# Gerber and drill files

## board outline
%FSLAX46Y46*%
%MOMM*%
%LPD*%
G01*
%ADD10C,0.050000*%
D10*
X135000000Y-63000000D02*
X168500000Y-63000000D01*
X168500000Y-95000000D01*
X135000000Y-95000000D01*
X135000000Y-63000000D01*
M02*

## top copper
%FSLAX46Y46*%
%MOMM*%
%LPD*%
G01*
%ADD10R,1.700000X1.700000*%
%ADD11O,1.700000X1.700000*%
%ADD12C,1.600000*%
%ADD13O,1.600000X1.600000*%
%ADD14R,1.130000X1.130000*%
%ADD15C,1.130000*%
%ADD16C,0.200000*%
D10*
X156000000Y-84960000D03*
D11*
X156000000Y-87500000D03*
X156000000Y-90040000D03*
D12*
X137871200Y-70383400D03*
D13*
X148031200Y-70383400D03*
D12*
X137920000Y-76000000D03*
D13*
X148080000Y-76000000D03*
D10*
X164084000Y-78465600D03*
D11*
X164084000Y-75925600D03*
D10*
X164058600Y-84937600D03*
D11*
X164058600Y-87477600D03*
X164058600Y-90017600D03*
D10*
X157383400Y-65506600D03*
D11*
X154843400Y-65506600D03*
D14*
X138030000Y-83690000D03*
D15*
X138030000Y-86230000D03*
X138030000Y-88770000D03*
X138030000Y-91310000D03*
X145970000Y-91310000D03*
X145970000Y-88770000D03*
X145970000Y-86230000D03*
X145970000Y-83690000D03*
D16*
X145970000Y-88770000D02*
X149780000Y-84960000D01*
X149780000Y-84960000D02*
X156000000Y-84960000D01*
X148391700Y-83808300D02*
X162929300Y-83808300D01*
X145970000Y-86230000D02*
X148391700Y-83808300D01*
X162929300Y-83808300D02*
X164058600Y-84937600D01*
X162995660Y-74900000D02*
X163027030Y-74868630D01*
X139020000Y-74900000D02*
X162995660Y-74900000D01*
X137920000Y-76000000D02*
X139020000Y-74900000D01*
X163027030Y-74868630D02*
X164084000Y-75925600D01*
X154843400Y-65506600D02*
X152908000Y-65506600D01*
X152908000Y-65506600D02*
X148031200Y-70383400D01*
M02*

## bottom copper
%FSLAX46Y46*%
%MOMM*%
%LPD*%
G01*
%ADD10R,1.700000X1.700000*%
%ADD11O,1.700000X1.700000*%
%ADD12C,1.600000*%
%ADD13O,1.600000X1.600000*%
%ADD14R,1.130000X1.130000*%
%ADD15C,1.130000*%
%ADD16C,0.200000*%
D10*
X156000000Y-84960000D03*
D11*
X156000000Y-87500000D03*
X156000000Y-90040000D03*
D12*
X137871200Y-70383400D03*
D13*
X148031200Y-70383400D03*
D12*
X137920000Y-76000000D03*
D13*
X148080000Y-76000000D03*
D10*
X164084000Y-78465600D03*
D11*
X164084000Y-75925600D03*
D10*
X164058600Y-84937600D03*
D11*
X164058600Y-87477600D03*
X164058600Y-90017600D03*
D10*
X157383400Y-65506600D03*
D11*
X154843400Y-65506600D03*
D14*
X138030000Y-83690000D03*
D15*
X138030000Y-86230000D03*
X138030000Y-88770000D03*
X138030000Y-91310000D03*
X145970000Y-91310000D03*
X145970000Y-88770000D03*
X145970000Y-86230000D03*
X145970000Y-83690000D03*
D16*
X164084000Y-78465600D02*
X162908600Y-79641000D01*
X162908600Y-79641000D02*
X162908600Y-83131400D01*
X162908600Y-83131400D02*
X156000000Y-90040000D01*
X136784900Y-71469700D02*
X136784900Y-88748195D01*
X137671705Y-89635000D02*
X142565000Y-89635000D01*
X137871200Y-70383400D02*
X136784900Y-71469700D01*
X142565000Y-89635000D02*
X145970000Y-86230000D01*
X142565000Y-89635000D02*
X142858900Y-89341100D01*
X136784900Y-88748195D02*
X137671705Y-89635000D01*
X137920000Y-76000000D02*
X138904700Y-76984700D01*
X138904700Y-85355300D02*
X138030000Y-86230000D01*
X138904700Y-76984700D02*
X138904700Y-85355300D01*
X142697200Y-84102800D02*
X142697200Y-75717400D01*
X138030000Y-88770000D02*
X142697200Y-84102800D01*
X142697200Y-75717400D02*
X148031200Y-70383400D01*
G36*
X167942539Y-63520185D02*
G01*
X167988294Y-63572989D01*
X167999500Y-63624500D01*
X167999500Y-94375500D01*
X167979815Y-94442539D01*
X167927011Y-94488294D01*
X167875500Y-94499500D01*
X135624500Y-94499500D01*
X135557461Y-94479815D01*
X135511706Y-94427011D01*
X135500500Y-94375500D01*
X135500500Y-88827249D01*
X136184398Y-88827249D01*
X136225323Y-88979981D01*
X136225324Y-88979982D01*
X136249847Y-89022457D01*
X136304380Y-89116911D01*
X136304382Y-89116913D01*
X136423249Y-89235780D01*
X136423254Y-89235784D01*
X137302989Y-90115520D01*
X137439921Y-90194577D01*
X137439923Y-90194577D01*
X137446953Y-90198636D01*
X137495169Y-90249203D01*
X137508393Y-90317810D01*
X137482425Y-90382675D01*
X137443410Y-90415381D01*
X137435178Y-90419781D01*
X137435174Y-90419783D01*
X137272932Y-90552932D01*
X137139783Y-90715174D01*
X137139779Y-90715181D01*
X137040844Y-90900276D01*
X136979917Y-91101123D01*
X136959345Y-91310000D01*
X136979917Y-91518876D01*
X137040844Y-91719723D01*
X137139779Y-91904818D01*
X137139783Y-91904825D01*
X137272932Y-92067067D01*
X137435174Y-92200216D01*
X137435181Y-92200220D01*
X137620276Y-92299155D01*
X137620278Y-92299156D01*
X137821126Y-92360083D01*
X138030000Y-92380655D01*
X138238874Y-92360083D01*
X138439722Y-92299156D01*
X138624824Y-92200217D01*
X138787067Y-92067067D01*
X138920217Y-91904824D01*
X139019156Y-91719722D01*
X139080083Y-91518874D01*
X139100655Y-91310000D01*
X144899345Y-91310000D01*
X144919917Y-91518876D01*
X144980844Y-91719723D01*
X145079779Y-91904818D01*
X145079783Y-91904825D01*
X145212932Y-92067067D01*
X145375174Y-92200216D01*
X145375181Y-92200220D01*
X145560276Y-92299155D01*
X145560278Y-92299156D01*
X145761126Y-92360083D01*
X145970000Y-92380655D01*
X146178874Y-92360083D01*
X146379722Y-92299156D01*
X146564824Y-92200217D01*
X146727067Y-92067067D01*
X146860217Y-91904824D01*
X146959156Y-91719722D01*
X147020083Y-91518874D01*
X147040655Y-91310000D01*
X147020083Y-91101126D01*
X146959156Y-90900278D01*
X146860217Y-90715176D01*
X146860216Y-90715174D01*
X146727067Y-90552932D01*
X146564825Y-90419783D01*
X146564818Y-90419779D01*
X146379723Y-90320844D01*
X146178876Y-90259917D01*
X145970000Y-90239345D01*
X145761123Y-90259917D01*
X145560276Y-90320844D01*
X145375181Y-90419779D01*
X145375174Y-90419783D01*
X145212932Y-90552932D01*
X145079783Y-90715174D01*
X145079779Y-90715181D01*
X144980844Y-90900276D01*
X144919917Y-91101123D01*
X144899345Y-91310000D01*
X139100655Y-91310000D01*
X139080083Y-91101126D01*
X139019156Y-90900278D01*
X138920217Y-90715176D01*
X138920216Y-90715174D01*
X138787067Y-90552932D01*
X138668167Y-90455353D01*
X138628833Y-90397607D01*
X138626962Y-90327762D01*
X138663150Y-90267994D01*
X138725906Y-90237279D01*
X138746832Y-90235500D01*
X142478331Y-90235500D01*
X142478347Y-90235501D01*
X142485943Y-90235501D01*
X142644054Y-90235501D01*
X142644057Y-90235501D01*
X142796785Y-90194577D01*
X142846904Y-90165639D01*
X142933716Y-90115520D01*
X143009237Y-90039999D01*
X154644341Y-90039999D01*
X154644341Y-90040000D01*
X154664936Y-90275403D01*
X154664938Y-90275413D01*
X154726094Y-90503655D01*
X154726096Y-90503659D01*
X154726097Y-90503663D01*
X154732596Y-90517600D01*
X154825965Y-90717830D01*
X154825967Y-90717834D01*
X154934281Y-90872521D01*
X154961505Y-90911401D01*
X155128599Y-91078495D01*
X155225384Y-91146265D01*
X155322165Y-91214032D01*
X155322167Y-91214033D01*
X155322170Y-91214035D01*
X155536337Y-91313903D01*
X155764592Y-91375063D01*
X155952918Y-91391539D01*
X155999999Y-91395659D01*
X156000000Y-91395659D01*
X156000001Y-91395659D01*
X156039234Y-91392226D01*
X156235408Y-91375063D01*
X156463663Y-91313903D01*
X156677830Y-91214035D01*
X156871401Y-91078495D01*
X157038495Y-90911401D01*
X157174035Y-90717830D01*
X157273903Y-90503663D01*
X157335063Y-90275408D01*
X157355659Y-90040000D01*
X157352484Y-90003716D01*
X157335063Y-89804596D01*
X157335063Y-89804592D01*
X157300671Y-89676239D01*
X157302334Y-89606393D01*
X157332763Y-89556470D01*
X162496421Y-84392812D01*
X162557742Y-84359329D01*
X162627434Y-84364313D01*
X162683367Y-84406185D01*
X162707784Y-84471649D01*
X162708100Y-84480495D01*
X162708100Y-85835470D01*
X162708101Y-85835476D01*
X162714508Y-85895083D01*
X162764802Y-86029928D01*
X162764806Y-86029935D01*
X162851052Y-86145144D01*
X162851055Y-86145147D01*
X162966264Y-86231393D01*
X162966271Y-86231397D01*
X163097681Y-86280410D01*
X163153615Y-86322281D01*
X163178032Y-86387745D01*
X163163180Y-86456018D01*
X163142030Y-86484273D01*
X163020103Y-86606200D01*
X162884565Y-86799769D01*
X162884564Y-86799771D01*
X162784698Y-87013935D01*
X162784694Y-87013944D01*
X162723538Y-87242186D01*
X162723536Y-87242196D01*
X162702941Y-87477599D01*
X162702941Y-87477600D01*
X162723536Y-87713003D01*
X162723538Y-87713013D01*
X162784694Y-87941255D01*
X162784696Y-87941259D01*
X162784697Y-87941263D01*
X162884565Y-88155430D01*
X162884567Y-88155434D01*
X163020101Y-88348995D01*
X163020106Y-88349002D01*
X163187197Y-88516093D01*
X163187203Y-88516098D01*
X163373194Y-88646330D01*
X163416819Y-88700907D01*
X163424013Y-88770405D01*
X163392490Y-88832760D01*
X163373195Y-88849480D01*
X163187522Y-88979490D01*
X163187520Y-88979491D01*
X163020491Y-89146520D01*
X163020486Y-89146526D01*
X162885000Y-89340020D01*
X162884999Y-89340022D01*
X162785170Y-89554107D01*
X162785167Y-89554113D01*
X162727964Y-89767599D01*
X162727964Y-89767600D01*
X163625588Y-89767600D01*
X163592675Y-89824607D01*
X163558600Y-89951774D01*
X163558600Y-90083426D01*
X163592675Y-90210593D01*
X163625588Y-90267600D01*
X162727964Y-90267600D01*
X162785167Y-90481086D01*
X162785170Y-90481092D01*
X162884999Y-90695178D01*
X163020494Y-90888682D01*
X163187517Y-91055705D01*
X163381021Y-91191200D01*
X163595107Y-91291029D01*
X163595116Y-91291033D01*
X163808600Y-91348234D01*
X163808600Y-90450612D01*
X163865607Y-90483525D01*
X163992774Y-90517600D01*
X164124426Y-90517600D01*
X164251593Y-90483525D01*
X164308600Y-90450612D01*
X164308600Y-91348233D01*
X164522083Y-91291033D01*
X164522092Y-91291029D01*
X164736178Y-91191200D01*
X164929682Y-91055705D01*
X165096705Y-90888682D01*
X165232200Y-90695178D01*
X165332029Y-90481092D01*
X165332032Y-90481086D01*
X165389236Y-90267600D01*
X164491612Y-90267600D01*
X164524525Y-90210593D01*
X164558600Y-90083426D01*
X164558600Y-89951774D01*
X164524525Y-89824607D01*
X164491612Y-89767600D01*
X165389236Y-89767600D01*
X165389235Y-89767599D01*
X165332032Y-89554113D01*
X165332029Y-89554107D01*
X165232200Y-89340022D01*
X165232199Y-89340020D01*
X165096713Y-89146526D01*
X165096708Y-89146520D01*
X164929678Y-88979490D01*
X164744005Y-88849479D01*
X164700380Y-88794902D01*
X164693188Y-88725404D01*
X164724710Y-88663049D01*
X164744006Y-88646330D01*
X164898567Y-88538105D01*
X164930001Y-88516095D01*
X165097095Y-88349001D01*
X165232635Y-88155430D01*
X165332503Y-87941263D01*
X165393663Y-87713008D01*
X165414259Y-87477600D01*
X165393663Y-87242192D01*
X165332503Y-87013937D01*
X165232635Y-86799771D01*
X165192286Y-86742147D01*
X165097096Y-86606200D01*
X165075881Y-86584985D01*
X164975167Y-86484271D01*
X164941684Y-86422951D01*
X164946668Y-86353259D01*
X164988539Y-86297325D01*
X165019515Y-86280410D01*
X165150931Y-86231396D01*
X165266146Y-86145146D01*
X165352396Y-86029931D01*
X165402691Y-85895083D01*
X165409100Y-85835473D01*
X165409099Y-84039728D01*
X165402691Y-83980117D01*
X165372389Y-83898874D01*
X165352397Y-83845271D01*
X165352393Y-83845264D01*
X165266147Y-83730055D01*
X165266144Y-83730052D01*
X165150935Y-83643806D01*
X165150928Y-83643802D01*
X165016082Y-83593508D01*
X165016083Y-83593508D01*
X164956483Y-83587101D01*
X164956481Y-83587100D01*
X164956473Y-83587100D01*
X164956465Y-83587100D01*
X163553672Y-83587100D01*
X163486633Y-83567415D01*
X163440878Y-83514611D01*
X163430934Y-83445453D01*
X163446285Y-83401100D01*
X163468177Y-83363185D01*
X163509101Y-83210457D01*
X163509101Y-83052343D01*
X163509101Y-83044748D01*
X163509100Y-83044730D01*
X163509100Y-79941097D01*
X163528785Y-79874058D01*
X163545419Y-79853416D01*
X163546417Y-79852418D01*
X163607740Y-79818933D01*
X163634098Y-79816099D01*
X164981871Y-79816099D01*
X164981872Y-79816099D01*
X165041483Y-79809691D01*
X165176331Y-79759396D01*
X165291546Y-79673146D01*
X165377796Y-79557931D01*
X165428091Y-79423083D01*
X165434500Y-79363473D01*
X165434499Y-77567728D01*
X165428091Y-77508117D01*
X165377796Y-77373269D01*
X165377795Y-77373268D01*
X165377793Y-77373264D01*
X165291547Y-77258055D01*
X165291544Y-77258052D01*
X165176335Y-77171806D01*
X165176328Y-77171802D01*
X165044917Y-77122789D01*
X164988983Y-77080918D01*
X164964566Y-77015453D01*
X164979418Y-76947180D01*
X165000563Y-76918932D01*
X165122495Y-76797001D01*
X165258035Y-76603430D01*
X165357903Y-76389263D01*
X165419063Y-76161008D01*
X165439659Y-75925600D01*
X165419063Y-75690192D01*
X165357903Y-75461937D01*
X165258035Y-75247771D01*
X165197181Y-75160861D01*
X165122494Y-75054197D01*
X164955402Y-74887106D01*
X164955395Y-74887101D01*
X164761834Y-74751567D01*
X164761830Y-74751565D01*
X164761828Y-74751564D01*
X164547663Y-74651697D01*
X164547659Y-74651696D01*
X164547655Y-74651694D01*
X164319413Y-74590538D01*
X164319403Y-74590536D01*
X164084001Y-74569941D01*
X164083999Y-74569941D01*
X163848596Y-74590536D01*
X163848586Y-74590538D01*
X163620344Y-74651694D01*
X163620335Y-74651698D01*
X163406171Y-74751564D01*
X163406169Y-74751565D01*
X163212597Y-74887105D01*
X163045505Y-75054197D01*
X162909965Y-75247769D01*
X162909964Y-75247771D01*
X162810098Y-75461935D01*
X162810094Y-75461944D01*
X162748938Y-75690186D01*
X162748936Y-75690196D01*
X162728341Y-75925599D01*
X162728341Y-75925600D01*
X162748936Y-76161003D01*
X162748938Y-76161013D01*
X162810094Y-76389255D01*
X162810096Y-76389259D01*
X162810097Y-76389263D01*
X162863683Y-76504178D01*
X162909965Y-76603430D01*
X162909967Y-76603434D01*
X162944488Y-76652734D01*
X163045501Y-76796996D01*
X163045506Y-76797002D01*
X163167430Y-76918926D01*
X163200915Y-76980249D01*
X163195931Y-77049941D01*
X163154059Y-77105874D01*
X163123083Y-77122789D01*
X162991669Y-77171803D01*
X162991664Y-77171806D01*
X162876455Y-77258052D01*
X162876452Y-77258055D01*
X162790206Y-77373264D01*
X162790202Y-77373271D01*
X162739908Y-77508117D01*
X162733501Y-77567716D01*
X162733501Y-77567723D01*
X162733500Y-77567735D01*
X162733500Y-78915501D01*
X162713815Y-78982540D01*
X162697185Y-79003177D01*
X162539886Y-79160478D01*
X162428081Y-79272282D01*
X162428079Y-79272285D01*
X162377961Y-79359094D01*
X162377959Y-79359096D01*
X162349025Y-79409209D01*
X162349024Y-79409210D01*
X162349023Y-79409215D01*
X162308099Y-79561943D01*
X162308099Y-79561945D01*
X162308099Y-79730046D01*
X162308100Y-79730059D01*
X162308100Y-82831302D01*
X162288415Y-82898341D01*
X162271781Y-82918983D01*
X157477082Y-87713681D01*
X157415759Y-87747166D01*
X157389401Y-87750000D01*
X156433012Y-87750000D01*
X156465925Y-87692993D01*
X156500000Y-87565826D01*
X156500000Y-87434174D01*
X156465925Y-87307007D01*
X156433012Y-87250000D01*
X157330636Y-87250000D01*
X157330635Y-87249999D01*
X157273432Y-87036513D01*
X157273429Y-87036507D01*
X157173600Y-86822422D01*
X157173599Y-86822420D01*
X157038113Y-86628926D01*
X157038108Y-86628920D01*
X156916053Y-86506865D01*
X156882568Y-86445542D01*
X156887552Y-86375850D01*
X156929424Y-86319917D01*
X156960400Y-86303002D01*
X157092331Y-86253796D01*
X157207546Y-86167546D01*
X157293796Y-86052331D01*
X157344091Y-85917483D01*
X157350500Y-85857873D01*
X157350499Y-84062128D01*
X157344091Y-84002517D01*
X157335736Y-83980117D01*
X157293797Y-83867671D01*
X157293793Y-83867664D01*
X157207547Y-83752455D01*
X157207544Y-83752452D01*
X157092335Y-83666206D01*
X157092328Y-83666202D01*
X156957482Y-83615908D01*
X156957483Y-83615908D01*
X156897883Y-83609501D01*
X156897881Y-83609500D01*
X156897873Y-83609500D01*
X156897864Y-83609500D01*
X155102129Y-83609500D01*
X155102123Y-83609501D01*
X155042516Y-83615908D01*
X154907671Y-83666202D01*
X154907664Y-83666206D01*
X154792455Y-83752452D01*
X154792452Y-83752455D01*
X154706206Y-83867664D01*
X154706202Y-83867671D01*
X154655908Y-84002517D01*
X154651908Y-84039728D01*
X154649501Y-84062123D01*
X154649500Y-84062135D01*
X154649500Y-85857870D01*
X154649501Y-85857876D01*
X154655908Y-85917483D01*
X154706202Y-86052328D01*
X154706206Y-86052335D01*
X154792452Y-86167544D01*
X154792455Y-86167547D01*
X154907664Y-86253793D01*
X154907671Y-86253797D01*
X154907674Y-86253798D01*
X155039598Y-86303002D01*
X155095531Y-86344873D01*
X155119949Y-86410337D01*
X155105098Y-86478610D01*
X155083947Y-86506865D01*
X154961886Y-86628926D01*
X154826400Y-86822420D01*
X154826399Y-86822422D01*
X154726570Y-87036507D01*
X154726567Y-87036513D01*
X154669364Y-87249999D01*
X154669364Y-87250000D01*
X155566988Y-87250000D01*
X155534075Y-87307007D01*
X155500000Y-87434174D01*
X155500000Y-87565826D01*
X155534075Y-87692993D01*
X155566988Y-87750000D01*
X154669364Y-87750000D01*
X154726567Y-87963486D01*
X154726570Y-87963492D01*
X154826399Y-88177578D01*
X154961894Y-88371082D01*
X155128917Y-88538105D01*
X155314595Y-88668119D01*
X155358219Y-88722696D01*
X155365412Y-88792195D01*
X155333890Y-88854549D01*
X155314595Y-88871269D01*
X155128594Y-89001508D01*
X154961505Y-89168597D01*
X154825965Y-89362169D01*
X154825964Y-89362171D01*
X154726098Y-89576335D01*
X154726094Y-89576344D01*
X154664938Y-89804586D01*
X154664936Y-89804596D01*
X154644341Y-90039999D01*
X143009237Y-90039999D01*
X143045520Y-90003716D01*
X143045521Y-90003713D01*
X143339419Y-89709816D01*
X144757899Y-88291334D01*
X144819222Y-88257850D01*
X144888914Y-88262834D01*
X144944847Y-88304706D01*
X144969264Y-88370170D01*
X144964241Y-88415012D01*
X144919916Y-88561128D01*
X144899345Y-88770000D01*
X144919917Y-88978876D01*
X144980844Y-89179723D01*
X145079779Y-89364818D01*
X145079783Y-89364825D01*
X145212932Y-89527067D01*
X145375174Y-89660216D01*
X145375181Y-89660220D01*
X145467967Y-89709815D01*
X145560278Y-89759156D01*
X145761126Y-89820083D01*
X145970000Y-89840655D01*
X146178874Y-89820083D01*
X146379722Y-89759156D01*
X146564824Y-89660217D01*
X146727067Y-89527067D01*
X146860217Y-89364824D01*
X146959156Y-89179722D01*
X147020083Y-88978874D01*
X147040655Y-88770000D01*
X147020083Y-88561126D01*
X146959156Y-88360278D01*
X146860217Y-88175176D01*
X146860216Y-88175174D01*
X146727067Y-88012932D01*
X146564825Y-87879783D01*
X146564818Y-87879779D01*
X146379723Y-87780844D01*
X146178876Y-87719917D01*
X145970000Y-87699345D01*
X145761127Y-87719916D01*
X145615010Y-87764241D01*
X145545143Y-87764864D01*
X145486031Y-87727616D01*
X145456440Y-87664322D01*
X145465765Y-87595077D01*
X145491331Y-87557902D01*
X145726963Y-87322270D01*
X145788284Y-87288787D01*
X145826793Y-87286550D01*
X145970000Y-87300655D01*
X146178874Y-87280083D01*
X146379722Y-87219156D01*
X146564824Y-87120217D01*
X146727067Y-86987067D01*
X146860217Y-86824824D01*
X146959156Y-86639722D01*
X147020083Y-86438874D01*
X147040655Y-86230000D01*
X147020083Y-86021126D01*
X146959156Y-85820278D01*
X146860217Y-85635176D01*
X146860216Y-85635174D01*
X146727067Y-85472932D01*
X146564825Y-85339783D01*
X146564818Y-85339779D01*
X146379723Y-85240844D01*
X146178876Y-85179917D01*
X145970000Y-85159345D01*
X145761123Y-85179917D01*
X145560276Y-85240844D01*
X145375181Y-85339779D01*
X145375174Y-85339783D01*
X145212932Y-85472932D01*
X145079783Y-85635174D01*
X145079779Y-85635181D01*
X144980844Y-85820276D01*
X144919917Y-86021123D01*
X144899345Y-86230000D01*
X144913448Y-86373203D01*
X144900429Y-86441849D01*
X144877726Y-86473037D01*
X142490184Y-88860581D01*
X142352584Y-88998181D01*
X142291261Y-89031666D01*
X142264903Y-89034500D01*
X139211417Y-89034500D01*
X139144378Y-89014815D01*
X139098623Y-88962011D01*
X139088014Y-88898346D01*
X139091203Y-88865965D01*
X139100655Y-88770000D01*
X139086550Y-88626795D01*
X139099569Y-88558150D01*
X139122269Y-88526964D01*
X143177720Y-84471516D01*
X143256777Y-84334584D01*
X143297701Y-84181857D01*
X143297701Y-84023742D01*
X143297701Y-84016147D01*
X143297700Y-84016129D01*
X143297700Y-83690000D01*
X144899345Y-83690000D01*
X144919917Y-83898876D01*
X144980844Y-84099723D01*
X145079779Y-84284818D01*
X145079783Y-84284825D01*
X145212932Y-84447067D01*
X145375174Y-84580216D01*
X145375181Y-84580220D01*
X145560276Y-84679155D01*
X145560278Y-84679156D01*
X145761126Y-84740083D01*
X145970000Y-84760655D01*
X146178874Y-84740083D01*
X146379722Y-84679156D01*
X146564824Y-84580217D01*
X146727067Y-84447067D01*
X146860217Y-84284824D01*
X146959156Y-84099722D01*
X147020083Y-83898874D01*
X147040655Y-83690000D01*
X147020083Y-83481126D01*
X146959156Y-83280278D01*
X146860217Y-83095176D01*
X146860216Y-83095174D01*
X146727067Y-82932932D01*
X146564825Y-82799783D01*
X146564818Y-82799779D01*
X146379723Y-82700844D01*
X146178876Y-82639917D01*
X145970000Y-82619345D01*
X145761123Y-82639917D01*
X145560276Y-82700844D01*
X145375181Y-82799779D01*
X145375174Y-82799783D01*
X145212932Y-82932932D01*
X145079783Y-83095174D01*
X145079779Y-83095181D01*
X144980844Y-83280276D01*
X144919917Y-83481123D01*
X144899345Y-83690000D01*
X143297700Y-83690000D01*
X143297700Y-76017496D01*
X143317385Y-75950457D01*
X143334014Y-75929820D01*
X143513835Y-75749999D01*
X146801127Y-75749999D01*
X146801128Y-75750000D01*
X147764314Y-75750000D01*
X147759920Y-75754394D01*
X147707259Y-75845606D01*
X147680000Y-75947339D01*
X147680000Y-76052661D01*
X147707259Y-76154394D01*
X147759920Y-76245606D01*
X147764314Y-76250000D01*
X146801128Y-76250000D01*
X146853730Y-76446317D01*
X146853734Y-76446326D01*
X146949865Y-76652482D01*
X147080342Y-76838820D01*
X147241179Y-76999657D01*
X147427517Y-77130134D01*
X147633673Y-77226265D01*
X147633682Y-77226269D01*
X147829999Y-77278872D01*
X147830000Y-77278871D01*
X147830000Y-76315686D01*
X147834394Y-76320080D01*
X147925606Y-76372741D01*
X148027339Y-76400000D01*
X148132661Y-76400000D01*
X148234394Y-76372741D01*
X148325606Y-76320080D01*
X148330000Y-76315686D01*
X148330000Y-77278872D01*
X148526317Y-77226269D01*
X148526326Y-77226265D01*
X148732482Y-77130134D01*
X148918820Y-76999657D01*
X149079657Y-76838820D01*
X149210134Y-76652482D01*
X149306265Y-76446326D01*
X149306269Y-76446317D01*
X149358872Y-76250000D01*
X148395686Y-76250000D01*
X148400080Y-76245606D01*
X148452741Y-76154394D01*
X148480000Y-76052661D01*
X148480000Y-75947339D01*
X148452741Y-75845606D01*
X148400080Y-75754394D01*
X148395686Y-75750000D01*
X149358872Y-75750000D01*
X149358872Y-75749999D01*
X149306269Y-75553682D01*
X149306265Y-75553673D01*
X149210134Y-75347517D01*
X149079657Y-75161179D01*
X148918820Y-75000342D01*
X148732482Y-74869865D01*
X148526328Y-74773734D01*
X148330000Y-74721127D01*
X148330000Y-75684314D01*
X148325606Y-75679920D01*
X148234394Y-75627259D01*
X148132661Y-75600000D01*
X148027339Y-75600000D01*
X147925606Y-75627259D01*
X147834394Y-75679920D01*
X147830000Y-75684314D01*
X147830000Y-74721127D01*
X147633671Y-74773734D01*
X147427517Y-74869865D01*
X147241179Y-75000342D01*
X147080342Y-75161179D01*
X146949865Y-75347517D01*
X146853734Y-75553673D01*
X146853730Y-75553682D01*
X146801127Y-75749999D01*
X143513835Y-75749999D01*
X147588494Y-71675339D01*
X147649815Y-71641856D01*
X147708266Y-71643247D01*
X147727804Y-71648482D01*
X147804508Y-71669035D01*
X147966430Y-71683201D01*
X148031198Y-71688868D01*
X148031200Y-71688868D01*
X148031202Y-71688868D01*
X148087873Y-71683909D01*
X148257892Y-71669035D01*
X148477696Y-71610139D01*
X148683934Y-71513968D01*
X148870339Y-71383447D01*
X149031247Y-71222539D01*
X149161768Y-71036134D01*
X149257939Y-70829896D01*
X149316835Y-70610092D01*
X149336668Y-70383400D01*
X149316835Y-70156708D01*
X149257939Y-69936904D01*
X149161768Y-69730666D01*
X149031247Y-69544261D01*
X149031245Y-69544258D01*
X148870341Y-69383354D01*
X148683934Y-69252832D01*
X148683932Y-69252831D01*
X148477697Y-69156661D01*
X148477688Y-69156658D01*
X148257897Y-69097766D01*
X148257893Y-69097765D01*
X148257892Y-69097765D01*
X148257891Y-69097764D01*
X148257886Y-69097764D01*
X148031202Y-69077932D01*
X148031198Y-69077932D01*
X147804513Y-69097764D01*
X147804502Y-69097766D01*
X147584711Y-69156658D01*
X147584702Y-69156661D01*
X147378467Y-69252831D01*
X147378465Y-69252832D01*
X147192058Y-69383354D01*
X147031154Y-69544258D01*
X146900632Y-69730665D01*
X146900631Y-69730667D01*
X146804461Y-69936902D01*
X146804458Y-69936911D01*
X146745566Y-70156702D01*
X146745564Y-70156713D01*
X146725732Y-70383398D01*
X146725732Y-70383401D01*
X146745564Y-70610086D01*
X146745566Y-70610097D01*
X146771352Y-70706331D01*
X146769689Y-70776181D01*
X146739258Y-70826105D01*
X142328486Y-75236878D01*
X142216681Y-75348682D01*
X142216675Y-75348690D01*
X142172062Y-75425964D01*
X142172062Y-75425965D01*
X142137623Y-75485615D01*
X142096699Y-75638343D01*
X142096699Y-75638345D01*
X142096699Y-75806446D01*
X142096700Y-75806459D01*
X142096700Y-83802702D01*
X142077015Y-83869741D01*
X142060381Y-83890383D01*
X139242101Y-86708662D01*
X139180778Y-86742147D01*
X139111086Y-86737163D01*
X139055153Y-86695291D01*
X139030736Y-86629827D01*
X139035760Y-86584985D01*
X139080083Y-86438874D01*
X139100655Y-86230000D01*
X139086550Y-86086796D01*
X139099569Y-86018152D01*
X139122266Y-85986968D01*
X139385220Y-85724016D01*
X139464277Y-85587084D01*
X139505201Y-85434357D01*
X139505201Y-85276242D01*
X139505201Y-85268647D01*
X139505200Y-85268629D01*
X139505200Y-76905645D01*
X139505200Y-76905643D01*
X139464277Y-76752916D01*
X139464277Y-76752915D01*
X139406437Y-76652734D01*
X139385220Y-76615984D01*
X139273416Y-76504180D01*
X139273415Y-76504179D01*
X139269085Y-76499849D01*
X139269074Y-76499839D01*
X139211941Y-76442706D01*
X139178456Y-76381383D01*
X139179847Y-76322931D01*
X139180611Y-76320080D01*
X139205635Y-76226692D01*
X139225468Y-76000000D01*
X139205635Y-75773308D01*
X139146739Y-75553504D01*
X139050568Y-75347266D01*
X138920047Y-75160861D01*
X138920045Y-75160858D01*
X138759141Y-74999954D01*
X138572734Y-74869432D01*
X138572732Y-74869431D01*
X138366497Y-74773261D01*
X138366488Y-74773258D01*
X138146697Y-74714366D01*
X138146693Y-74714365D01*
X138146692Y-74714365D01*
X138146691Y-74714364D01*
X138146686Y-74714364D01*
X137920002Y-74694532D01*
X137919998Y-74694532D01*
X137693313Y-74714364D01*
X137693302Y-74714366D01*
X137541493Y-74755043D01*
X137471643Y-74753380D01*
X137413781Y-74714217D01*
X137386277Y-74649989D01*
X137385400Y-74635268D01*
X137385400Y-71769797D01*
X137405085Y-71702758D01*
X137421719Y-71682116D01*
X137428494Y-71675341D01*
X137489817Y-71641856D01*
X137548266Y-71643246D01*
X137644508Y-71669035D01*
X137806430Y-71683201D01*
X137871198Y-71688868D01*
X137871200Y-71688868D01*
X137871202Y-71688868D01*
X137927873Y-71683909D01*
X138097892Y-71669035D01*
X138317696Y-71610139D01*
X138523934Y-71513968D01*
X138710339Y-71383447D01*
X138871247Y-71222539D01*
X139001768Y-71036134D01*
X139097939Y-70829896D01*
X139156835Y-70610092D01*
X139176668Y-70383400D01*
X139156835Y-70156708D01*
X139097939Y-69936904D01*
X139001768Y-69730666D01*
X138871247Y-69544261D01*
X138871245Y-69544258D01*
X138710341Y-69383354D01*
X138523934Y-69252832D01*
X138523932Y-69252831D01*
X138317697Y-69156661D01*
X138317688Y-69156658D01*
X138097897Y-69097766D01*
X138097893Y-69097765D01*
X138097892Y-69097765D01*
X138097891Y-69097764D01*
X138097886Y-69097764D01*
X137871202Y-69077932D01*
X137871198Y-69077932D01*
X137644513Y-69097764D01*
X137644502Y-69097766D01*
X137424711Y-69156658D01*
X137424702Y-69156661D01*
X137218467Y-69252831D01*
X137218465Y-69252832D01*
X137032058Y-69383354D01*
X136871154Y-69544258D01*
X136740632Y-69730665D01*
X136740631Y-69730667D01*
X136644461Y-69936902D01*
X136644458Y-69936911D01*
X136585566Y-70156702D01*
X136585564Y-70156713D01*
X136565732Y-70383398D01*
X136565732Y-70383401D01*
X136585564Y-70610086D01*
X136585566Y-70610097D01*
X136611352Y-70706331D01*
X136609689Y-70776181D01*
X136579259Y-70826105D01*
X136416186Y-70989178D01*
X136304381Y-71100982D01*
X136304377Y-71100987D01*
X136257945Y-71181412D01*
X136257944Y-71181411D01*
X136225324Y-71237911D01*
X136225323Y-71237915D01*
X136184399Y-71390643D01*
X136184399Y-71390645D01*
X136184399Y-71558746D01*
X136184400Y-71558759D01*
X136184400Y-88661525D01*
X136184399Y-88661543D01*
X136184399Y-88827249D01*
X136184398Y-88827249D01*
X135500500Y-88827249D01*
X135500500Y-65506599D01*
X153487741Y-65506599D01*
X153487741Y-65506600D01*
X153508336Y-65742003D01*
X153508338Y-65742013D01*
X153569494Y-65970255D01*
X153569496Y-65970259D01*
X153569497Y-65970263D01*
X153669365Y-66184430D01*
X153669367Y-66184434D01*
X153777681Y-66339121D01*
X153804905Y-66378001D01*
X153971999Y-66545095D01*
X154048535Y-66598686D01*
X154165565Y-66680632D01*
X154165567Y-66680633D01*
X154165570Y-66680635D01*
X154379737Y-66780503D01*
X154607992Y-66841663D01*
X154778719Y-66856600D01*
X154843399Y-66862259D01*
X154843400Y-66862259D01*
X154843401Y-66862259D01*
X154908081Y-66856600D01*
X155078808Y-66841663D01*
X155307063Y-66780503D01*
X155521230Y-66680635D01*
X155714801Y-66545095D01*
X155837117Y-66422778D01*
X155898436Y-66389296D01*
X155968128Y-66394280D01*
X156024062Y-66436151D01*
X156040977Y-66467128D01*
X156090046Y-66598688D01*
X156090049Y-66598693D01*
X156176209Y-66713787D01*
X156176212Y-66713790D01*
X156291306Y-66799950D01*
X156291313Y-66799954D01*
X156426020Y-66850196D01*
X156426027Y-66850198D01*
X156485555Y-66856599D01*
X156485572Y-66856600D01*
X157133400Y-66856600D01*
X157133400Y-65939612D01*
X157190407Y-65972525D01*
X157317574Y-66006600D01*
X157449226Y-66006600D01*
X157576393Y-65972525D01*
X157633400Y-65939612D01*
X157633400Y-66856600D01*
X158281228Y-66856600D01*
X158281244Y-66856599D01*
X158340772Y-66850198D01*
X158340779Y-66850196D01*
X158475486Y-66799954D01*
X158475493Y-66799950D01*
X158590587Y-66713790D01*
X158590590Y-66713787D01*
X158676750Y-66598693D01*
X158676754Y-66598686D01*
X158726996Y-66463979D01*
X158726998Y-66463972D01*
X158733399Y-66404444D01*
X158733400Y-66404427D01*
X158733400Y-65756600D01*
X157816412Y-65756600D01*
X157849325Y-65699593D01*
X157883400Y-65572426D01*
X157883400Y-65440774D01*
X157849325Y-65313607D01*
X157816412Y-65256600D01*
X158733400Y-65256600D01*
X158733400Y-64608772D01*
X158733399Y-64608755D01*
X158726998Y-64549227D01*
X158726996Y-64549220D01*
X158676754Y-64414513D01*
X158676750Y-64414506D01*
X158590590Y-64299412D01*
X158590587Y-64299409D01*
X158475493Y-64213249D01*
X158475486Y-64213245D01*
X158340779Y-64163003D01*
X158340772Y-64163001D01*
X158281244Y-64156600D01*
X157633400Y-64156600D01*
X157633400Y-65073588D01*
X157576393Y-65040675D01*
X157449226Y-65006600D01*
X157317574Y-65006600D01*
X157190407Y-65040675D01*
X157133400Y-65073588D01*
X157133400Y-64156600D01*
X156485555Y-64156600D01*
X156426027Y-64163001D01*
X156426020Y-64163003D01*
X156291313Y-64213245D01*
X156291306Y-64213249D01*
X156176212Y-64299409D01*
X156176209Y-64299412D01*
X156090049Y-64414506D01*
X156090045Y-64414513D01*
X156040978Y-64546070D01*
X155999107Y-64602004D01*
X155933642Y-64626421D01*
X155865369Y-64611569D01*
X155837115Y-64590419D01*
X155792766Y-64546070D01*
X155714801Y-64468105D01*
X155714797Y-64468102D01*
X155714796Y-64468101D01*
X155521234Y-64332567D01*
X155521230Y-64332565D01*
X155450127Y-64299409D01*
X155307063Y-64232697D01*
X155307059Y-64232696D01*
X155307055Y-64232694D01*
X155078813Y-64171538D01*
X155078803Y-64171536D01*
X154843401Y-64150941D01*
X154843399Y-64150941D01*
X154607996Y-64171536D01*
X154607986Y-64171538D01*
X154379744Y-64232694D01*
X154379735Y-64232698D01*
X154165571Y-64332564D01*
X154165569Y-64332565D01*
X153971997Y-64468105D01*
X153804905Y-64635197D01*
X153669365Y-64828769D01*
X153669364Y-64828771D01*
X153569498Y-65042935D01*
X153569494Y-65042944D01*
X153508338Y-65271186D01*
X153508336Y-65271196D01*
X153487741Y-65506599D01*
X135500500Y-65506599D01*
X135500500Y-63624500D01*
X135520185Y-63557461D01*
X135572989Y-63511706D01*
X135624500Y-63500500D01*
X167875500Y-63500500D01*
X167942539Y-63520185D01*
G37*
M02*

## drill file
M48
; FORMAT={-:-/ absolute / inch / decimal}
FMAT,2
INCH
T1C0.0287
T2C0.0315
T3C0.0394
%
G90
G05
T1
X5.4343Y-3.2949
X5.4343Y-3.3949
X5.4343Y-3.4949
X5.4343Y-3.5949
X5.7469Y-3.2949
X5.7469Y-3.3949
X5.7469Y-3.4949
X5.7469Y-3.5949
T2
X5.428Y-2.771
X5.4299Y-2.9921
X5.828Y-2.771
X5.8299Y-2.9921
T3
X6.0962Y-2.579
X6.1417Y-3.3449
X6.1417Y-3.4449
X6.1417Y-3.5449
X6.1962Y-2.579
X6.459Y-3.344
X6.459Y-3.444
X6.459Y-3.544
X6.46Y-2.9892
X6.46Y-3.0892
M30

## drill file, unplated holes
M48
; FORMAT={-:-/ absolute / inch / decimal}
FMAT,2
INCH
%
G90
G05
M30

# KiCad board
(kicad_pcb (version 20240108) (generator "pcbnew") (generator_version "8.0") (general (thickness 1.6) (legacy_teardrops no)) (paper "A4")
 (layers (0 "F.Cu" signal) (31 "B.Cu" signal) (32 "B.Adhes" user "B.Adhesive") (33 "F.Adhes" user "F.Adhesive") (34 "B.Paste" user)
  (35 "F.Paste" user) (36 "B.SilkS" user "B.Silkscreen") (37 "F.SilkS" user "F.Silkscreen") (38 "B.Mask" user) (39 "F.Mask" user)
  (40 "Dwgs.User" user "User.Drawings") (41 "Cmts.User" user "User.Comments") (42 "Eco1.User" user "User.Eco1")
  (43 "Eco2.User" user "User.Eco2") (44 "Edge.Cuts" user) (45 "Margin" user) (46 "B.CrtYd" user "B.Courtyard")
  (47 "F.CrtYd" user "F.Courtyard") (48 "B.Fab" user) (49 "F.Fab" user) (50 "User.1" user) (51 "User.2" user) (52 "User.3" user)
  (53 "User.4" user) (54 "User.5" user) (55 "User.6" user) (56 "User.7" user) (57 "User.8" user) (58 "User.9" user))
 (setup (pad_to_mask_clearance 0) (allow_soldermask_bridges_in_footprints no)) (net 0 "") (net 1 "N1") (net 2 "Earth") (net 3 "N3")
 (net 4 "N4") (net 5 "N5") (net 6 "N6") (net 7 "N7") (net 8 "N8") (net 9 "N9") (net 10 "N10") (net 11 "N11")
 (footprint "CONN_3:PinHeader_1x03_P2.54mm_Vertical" (layer "F.Cu") (at 156 84.96)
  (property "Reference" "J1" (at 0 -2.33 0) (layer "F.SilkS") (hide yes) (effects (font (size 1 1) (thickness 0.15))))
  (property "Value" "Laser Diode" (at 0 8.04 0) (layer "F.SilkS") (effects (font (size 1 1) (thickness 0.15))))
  (pad "1" thru_hole rect (at 0 0) (size 1.7 1.7) (drill 1) (layers "*.Cu" "*.Mask") (remove_unused_layers no) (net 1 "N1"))
  (pad "2" thru_hole oval (at 0 2.54) (size 1.7 1.7) (drill 1) (layers "*.Cu" "*.Mask") (remove_unused_layers no) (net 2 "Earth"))
  (pad "3" thru_hole oval (at 0 5.08) (size 1.7 1.7) (drill 1) (layers "*.Cu" "*.Mask") (remove_unused_layers no) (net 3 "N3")))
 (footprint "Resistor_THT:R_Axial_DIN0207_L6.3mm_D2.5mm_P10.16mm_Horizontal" (layer "F.Cu") (at 137.8712 70.3834)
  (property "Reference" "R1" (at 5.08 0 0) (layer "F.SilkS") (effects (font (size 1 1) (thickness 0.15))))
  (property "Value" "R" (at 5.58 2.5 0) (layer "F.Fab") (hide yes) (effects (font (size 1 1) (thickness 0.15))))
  (pad "1" thru_hole circle (at 0 0) (size 1.6 1.6) (drill 0.8) (layers "*.Cu" "*.Mask") (remove_unused_layers no) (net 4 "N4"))
  (pad "2" thru_hole oval (at 10.16 0) (size 1.6 1.6) (drill 0.8) (layers "*.Cu" "*.Mask") (remove_unused_layers no) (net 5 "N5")))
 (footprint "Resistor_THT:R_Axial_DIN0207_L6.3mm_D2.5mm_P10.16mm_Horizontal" (layer "F.Cu") (at 137.92 76)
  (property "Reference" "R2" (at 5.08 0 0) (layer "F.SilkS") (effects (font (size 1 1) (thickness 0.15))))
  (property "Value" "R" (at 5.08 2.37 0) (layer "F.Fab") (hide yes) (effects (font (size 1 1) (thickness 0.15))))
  (pad "1" thru_hole circle (at 0 0) (size 1.6 1.6) (drill 0.8) (layers "*.Cu" "*.Mask") (remove_unused_layers no) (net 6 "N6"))
  (pad "2" thru_hole oval (at 10.16 0) (size 1.6 1.6) (drill 0.8) (layers "*.Cu" "*.Mask") (remove_unused_layers no) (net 2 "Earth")))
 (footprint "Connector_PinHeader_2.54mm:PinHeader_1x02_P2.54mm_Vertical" (layer "F.Cu") (at 164.084 78.4656 180)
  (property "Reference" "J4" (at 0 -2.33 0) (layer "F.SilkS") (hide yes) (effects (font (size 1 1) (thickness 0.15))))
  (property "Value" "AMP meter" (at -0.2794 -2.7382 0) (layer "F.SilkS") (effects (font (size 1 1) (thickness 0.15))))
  (pad "1" thru_hole rect (at 0 0 180) (size 1.7 1.7) (drill 1) (layers "*.Cu" "*.Mask") (remove_unused_layers no) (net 3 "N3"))
  (pad "2" thru_hole oval (at 0 2.54 180) (size 1.7 1.7) (drill 1) (layers "*.Cu" "*.Mask") (remove_unused_layers no) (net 6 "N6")))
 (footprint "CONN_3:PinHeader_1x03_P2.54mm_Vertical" (layer "F.Cu") (at 164.0586 84.9376)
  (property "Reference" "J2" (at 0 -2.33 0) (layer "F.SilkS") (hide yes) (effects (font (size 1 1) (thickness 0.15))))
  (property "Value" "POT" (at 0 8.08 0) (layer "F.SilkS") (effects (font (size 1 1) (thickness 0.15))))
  (pad "1" thru_hole rect (at 0 0) (size 1.7 1.7) (drill 1) (layers "*.Cu" "*.Mask") (remove_unused_layers no) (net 4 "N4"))
  (pad "2" thru_hole oval (at 0 2.54) (size 1.7 1.7) (drill 1) (layers "*.Cu" "*.Mask") (remove_unused_layers no) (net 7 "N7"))
  (pad "3" thru_hole oval (at 0 5.08) (size 1.7 1.7) (drill 1) (layers "*.Cu" "*.Mask") (remove_unused_layers no) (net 2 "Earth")))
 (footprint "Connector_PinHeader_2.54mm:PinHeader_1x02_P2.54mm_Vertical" (layer "F.Cu") (at 157.3834 65.5066 -90)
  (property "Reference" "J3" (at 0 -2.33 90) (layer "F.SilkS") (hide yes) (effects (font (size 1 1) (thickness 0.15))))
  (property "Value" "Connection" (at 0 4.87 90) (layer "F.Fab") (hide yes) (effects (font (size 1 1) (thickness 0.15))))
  (pad "1" thru_hole rect (at 0 0 270) (size 1.7 1.7) (drill 1) (layers "*.Cu" "*.Mask") (remove_unused_layers no) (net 2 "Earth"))
  (pad "2" thru_hole oval (at 0 2.54 270) (size 1.7 1.7) (drill 1) (layers "*.Cu" "*.Mask") (remove_unused_layers no) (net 5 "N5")))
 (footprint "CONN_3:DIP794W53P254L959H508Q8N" (layer "F.Cu") (at 142 87.5)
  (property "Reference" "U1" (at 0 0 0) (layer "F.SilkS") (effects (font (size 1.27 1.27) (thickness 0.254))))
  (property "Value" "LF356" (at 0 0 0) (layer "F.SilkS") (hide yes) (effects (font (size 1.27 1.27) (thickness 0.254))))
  (pad "1" thru_hole rect (at -3.97 -3.81) (size 1.13 1.13) (drill 0.73) (layers "*.Cu" "*.Mask") (remove_unused_layers no) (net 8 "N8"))
  (pad "2" thru_hole circle (at -3.97 -1.27) (size 1.13 1.13) (drill 0.73) (layers "*.Cu" "*.Mask") (remove_unused_layers no) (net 6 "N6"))
  (pad "3" thru_hole circle (at -3.97 1.27) (size 1.13 1.13) (drill 0.73) (layers "*.Cu" "*.Mask") (remove_unused_layers no) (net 5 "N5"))
  (pad "4" thru_hole circle (at -3.97 3.81) (size 1.13 1.13) (drill 0.73) (layers "*.Cu" "*.Mask") (remove_unused_layers no) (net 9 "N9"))
  (pad "5" thru_hole circle (at 3.97 3.81) (size 1.13 1.13) (drill 0.73) (layers "*.Cu" "*.Mask") (remove_unused_layers no) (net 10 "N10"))
  (pad "6" thru_hole circle (at 3.97 1.27) (size 1.13 1.13) (drill 0.73) (layers "*.Cu" "*.Mask") (remove_unused_layers no) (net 1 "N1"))
  (pad "7" thru_hole circle (at 3.97 -1.27) (size 1.13 1.13) (drill 0.73) (layers "*.Cu" "*.Mask") (remove_unused_layers no) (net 4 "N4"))
  (pad "8" thru_hole circle (at 3.97 -3.81) (size 1.13 1.13) (drill 0.73) (layers "*.Cu" "*.Mask") (remove_unused_layers no) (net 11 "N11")))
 (gr_rect (start 135 63) (end 168.5 95) (stroke (width 0.05) (type default)) (fill none) (layer "Edge.Cuts"))
 (segment (start 164.084 78.4656) (end 162.9086 79.641) (width 0.2) (layer "B.Cu") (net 3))
 (segment (start 162.9086 79.641) (end 162.9086 83.1314) (width 0.2) (layer "B.Cu") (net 3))
 (segment (start 162.9086 83.1314) (end 156 90.04) (width 0.2) (layer "B.Cu") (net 3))
 (segment (start 145.97 88.77) (end 149.78 84.96) (width 0.2) (layer "F.Cu") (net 1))
 (segment (start 149.78 84.96) (end 156 84.96) (width 0.2) (layer "F.Cu") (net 1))
 (segment (start 148.3917 83.8083) (end 162.9293 83.8083) (width 0.2) (layer "F.Cu") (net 4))
 (segment (start 145.97 86.23) (end 148.3917 83.8083) (width 0.2) (layer "F.Cu") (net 4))
 (segment (start 162.9293 83.8083) (end 164.0586 84.9376) (width 0.2) (layer "F.Cu") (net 4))
 (segment (start 136.7849 71.4697) (end 136.7849 88.748195) (width 0.2) (layer "B.Cu") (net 4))
 (segment (start 137.671705 89.635) (end 142.565 89.635) (width 0.2) (layer "B.Cu") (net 4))
 (segment (start 137.8712 70.3834) (end 136.7849 71.4697) (width 0.2) (layer "B.Cu") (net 4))
 (segment (start 142.565 89.635) (end 145.97 86.23) (width 0.2) (layer "B.Cu") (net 4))
 (segment (start 142.565 89.635) (end 142.8589 89.3411) (width 0.2) (layer "B.Cu") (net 4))
 (segment (start 136.7849 88.748195) (end 137.671705 89.635) (width 0.2) (layer "B.Cu") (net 4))
 (segment (start 162.99566 74.9) (end 163.02703 74.86863) (width 0.2) (layer "F.Cu") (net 6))
 (segment (start 139.02 74.9) (end 162.99566 74.9) (width 0.2) (layer "F.Cu") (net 6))
 (segment (start 137.92 76) (end 139.02 74.9) (width 0.2) (layer "F.Cu") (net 6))
 (segment (start 163.02703 74.86863) (end 164.084 75.9256) (width 0.2) (layer "F.Cu") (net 6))
 (segment (start 137.92 76) (end 138.9047 76.9847) (width 0.2) (layer "B.Cu") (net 6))
 (segment (start 138.9047 85.3553) (end 138.03 86.23) (width 0.2) (layer "B.Cu") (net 6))
 (segment (start 138.9047 76.9847) (end 138.9047 85.3553) (width 0.2) (layer "B.Cu") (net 6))
 (segment (start 154.8434 65.5066) (end 152.908 65.5066) (width 0.2) (layer "F.Cu") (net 5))
 (segment (start 152.908 65.5066) (end 148.0312 70.3834) (width 0.2) (layer "F.Cu") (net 5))
 (segment (start 142.6972 84.1028) (end 142.6972 75.7174) (width 0.2) (layer "B.Cu") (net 5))
 (segment (start 138.03 88.77) (end 142.6972 84.1028) (width 0.2) (layer "B.Cu") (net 5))
 (segment (start 142.6972 75.7174) (end 148.0312 70.3834) (width 0.2) (layer "B.Cu") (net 5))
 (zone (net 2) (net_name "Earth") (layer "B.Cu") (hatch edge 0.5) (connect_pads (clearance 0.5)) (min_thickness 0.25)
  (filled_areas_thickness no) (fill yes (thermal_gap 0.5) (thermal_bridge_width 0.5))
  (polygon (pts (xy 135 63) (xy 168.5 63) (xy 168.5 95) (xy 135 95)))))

